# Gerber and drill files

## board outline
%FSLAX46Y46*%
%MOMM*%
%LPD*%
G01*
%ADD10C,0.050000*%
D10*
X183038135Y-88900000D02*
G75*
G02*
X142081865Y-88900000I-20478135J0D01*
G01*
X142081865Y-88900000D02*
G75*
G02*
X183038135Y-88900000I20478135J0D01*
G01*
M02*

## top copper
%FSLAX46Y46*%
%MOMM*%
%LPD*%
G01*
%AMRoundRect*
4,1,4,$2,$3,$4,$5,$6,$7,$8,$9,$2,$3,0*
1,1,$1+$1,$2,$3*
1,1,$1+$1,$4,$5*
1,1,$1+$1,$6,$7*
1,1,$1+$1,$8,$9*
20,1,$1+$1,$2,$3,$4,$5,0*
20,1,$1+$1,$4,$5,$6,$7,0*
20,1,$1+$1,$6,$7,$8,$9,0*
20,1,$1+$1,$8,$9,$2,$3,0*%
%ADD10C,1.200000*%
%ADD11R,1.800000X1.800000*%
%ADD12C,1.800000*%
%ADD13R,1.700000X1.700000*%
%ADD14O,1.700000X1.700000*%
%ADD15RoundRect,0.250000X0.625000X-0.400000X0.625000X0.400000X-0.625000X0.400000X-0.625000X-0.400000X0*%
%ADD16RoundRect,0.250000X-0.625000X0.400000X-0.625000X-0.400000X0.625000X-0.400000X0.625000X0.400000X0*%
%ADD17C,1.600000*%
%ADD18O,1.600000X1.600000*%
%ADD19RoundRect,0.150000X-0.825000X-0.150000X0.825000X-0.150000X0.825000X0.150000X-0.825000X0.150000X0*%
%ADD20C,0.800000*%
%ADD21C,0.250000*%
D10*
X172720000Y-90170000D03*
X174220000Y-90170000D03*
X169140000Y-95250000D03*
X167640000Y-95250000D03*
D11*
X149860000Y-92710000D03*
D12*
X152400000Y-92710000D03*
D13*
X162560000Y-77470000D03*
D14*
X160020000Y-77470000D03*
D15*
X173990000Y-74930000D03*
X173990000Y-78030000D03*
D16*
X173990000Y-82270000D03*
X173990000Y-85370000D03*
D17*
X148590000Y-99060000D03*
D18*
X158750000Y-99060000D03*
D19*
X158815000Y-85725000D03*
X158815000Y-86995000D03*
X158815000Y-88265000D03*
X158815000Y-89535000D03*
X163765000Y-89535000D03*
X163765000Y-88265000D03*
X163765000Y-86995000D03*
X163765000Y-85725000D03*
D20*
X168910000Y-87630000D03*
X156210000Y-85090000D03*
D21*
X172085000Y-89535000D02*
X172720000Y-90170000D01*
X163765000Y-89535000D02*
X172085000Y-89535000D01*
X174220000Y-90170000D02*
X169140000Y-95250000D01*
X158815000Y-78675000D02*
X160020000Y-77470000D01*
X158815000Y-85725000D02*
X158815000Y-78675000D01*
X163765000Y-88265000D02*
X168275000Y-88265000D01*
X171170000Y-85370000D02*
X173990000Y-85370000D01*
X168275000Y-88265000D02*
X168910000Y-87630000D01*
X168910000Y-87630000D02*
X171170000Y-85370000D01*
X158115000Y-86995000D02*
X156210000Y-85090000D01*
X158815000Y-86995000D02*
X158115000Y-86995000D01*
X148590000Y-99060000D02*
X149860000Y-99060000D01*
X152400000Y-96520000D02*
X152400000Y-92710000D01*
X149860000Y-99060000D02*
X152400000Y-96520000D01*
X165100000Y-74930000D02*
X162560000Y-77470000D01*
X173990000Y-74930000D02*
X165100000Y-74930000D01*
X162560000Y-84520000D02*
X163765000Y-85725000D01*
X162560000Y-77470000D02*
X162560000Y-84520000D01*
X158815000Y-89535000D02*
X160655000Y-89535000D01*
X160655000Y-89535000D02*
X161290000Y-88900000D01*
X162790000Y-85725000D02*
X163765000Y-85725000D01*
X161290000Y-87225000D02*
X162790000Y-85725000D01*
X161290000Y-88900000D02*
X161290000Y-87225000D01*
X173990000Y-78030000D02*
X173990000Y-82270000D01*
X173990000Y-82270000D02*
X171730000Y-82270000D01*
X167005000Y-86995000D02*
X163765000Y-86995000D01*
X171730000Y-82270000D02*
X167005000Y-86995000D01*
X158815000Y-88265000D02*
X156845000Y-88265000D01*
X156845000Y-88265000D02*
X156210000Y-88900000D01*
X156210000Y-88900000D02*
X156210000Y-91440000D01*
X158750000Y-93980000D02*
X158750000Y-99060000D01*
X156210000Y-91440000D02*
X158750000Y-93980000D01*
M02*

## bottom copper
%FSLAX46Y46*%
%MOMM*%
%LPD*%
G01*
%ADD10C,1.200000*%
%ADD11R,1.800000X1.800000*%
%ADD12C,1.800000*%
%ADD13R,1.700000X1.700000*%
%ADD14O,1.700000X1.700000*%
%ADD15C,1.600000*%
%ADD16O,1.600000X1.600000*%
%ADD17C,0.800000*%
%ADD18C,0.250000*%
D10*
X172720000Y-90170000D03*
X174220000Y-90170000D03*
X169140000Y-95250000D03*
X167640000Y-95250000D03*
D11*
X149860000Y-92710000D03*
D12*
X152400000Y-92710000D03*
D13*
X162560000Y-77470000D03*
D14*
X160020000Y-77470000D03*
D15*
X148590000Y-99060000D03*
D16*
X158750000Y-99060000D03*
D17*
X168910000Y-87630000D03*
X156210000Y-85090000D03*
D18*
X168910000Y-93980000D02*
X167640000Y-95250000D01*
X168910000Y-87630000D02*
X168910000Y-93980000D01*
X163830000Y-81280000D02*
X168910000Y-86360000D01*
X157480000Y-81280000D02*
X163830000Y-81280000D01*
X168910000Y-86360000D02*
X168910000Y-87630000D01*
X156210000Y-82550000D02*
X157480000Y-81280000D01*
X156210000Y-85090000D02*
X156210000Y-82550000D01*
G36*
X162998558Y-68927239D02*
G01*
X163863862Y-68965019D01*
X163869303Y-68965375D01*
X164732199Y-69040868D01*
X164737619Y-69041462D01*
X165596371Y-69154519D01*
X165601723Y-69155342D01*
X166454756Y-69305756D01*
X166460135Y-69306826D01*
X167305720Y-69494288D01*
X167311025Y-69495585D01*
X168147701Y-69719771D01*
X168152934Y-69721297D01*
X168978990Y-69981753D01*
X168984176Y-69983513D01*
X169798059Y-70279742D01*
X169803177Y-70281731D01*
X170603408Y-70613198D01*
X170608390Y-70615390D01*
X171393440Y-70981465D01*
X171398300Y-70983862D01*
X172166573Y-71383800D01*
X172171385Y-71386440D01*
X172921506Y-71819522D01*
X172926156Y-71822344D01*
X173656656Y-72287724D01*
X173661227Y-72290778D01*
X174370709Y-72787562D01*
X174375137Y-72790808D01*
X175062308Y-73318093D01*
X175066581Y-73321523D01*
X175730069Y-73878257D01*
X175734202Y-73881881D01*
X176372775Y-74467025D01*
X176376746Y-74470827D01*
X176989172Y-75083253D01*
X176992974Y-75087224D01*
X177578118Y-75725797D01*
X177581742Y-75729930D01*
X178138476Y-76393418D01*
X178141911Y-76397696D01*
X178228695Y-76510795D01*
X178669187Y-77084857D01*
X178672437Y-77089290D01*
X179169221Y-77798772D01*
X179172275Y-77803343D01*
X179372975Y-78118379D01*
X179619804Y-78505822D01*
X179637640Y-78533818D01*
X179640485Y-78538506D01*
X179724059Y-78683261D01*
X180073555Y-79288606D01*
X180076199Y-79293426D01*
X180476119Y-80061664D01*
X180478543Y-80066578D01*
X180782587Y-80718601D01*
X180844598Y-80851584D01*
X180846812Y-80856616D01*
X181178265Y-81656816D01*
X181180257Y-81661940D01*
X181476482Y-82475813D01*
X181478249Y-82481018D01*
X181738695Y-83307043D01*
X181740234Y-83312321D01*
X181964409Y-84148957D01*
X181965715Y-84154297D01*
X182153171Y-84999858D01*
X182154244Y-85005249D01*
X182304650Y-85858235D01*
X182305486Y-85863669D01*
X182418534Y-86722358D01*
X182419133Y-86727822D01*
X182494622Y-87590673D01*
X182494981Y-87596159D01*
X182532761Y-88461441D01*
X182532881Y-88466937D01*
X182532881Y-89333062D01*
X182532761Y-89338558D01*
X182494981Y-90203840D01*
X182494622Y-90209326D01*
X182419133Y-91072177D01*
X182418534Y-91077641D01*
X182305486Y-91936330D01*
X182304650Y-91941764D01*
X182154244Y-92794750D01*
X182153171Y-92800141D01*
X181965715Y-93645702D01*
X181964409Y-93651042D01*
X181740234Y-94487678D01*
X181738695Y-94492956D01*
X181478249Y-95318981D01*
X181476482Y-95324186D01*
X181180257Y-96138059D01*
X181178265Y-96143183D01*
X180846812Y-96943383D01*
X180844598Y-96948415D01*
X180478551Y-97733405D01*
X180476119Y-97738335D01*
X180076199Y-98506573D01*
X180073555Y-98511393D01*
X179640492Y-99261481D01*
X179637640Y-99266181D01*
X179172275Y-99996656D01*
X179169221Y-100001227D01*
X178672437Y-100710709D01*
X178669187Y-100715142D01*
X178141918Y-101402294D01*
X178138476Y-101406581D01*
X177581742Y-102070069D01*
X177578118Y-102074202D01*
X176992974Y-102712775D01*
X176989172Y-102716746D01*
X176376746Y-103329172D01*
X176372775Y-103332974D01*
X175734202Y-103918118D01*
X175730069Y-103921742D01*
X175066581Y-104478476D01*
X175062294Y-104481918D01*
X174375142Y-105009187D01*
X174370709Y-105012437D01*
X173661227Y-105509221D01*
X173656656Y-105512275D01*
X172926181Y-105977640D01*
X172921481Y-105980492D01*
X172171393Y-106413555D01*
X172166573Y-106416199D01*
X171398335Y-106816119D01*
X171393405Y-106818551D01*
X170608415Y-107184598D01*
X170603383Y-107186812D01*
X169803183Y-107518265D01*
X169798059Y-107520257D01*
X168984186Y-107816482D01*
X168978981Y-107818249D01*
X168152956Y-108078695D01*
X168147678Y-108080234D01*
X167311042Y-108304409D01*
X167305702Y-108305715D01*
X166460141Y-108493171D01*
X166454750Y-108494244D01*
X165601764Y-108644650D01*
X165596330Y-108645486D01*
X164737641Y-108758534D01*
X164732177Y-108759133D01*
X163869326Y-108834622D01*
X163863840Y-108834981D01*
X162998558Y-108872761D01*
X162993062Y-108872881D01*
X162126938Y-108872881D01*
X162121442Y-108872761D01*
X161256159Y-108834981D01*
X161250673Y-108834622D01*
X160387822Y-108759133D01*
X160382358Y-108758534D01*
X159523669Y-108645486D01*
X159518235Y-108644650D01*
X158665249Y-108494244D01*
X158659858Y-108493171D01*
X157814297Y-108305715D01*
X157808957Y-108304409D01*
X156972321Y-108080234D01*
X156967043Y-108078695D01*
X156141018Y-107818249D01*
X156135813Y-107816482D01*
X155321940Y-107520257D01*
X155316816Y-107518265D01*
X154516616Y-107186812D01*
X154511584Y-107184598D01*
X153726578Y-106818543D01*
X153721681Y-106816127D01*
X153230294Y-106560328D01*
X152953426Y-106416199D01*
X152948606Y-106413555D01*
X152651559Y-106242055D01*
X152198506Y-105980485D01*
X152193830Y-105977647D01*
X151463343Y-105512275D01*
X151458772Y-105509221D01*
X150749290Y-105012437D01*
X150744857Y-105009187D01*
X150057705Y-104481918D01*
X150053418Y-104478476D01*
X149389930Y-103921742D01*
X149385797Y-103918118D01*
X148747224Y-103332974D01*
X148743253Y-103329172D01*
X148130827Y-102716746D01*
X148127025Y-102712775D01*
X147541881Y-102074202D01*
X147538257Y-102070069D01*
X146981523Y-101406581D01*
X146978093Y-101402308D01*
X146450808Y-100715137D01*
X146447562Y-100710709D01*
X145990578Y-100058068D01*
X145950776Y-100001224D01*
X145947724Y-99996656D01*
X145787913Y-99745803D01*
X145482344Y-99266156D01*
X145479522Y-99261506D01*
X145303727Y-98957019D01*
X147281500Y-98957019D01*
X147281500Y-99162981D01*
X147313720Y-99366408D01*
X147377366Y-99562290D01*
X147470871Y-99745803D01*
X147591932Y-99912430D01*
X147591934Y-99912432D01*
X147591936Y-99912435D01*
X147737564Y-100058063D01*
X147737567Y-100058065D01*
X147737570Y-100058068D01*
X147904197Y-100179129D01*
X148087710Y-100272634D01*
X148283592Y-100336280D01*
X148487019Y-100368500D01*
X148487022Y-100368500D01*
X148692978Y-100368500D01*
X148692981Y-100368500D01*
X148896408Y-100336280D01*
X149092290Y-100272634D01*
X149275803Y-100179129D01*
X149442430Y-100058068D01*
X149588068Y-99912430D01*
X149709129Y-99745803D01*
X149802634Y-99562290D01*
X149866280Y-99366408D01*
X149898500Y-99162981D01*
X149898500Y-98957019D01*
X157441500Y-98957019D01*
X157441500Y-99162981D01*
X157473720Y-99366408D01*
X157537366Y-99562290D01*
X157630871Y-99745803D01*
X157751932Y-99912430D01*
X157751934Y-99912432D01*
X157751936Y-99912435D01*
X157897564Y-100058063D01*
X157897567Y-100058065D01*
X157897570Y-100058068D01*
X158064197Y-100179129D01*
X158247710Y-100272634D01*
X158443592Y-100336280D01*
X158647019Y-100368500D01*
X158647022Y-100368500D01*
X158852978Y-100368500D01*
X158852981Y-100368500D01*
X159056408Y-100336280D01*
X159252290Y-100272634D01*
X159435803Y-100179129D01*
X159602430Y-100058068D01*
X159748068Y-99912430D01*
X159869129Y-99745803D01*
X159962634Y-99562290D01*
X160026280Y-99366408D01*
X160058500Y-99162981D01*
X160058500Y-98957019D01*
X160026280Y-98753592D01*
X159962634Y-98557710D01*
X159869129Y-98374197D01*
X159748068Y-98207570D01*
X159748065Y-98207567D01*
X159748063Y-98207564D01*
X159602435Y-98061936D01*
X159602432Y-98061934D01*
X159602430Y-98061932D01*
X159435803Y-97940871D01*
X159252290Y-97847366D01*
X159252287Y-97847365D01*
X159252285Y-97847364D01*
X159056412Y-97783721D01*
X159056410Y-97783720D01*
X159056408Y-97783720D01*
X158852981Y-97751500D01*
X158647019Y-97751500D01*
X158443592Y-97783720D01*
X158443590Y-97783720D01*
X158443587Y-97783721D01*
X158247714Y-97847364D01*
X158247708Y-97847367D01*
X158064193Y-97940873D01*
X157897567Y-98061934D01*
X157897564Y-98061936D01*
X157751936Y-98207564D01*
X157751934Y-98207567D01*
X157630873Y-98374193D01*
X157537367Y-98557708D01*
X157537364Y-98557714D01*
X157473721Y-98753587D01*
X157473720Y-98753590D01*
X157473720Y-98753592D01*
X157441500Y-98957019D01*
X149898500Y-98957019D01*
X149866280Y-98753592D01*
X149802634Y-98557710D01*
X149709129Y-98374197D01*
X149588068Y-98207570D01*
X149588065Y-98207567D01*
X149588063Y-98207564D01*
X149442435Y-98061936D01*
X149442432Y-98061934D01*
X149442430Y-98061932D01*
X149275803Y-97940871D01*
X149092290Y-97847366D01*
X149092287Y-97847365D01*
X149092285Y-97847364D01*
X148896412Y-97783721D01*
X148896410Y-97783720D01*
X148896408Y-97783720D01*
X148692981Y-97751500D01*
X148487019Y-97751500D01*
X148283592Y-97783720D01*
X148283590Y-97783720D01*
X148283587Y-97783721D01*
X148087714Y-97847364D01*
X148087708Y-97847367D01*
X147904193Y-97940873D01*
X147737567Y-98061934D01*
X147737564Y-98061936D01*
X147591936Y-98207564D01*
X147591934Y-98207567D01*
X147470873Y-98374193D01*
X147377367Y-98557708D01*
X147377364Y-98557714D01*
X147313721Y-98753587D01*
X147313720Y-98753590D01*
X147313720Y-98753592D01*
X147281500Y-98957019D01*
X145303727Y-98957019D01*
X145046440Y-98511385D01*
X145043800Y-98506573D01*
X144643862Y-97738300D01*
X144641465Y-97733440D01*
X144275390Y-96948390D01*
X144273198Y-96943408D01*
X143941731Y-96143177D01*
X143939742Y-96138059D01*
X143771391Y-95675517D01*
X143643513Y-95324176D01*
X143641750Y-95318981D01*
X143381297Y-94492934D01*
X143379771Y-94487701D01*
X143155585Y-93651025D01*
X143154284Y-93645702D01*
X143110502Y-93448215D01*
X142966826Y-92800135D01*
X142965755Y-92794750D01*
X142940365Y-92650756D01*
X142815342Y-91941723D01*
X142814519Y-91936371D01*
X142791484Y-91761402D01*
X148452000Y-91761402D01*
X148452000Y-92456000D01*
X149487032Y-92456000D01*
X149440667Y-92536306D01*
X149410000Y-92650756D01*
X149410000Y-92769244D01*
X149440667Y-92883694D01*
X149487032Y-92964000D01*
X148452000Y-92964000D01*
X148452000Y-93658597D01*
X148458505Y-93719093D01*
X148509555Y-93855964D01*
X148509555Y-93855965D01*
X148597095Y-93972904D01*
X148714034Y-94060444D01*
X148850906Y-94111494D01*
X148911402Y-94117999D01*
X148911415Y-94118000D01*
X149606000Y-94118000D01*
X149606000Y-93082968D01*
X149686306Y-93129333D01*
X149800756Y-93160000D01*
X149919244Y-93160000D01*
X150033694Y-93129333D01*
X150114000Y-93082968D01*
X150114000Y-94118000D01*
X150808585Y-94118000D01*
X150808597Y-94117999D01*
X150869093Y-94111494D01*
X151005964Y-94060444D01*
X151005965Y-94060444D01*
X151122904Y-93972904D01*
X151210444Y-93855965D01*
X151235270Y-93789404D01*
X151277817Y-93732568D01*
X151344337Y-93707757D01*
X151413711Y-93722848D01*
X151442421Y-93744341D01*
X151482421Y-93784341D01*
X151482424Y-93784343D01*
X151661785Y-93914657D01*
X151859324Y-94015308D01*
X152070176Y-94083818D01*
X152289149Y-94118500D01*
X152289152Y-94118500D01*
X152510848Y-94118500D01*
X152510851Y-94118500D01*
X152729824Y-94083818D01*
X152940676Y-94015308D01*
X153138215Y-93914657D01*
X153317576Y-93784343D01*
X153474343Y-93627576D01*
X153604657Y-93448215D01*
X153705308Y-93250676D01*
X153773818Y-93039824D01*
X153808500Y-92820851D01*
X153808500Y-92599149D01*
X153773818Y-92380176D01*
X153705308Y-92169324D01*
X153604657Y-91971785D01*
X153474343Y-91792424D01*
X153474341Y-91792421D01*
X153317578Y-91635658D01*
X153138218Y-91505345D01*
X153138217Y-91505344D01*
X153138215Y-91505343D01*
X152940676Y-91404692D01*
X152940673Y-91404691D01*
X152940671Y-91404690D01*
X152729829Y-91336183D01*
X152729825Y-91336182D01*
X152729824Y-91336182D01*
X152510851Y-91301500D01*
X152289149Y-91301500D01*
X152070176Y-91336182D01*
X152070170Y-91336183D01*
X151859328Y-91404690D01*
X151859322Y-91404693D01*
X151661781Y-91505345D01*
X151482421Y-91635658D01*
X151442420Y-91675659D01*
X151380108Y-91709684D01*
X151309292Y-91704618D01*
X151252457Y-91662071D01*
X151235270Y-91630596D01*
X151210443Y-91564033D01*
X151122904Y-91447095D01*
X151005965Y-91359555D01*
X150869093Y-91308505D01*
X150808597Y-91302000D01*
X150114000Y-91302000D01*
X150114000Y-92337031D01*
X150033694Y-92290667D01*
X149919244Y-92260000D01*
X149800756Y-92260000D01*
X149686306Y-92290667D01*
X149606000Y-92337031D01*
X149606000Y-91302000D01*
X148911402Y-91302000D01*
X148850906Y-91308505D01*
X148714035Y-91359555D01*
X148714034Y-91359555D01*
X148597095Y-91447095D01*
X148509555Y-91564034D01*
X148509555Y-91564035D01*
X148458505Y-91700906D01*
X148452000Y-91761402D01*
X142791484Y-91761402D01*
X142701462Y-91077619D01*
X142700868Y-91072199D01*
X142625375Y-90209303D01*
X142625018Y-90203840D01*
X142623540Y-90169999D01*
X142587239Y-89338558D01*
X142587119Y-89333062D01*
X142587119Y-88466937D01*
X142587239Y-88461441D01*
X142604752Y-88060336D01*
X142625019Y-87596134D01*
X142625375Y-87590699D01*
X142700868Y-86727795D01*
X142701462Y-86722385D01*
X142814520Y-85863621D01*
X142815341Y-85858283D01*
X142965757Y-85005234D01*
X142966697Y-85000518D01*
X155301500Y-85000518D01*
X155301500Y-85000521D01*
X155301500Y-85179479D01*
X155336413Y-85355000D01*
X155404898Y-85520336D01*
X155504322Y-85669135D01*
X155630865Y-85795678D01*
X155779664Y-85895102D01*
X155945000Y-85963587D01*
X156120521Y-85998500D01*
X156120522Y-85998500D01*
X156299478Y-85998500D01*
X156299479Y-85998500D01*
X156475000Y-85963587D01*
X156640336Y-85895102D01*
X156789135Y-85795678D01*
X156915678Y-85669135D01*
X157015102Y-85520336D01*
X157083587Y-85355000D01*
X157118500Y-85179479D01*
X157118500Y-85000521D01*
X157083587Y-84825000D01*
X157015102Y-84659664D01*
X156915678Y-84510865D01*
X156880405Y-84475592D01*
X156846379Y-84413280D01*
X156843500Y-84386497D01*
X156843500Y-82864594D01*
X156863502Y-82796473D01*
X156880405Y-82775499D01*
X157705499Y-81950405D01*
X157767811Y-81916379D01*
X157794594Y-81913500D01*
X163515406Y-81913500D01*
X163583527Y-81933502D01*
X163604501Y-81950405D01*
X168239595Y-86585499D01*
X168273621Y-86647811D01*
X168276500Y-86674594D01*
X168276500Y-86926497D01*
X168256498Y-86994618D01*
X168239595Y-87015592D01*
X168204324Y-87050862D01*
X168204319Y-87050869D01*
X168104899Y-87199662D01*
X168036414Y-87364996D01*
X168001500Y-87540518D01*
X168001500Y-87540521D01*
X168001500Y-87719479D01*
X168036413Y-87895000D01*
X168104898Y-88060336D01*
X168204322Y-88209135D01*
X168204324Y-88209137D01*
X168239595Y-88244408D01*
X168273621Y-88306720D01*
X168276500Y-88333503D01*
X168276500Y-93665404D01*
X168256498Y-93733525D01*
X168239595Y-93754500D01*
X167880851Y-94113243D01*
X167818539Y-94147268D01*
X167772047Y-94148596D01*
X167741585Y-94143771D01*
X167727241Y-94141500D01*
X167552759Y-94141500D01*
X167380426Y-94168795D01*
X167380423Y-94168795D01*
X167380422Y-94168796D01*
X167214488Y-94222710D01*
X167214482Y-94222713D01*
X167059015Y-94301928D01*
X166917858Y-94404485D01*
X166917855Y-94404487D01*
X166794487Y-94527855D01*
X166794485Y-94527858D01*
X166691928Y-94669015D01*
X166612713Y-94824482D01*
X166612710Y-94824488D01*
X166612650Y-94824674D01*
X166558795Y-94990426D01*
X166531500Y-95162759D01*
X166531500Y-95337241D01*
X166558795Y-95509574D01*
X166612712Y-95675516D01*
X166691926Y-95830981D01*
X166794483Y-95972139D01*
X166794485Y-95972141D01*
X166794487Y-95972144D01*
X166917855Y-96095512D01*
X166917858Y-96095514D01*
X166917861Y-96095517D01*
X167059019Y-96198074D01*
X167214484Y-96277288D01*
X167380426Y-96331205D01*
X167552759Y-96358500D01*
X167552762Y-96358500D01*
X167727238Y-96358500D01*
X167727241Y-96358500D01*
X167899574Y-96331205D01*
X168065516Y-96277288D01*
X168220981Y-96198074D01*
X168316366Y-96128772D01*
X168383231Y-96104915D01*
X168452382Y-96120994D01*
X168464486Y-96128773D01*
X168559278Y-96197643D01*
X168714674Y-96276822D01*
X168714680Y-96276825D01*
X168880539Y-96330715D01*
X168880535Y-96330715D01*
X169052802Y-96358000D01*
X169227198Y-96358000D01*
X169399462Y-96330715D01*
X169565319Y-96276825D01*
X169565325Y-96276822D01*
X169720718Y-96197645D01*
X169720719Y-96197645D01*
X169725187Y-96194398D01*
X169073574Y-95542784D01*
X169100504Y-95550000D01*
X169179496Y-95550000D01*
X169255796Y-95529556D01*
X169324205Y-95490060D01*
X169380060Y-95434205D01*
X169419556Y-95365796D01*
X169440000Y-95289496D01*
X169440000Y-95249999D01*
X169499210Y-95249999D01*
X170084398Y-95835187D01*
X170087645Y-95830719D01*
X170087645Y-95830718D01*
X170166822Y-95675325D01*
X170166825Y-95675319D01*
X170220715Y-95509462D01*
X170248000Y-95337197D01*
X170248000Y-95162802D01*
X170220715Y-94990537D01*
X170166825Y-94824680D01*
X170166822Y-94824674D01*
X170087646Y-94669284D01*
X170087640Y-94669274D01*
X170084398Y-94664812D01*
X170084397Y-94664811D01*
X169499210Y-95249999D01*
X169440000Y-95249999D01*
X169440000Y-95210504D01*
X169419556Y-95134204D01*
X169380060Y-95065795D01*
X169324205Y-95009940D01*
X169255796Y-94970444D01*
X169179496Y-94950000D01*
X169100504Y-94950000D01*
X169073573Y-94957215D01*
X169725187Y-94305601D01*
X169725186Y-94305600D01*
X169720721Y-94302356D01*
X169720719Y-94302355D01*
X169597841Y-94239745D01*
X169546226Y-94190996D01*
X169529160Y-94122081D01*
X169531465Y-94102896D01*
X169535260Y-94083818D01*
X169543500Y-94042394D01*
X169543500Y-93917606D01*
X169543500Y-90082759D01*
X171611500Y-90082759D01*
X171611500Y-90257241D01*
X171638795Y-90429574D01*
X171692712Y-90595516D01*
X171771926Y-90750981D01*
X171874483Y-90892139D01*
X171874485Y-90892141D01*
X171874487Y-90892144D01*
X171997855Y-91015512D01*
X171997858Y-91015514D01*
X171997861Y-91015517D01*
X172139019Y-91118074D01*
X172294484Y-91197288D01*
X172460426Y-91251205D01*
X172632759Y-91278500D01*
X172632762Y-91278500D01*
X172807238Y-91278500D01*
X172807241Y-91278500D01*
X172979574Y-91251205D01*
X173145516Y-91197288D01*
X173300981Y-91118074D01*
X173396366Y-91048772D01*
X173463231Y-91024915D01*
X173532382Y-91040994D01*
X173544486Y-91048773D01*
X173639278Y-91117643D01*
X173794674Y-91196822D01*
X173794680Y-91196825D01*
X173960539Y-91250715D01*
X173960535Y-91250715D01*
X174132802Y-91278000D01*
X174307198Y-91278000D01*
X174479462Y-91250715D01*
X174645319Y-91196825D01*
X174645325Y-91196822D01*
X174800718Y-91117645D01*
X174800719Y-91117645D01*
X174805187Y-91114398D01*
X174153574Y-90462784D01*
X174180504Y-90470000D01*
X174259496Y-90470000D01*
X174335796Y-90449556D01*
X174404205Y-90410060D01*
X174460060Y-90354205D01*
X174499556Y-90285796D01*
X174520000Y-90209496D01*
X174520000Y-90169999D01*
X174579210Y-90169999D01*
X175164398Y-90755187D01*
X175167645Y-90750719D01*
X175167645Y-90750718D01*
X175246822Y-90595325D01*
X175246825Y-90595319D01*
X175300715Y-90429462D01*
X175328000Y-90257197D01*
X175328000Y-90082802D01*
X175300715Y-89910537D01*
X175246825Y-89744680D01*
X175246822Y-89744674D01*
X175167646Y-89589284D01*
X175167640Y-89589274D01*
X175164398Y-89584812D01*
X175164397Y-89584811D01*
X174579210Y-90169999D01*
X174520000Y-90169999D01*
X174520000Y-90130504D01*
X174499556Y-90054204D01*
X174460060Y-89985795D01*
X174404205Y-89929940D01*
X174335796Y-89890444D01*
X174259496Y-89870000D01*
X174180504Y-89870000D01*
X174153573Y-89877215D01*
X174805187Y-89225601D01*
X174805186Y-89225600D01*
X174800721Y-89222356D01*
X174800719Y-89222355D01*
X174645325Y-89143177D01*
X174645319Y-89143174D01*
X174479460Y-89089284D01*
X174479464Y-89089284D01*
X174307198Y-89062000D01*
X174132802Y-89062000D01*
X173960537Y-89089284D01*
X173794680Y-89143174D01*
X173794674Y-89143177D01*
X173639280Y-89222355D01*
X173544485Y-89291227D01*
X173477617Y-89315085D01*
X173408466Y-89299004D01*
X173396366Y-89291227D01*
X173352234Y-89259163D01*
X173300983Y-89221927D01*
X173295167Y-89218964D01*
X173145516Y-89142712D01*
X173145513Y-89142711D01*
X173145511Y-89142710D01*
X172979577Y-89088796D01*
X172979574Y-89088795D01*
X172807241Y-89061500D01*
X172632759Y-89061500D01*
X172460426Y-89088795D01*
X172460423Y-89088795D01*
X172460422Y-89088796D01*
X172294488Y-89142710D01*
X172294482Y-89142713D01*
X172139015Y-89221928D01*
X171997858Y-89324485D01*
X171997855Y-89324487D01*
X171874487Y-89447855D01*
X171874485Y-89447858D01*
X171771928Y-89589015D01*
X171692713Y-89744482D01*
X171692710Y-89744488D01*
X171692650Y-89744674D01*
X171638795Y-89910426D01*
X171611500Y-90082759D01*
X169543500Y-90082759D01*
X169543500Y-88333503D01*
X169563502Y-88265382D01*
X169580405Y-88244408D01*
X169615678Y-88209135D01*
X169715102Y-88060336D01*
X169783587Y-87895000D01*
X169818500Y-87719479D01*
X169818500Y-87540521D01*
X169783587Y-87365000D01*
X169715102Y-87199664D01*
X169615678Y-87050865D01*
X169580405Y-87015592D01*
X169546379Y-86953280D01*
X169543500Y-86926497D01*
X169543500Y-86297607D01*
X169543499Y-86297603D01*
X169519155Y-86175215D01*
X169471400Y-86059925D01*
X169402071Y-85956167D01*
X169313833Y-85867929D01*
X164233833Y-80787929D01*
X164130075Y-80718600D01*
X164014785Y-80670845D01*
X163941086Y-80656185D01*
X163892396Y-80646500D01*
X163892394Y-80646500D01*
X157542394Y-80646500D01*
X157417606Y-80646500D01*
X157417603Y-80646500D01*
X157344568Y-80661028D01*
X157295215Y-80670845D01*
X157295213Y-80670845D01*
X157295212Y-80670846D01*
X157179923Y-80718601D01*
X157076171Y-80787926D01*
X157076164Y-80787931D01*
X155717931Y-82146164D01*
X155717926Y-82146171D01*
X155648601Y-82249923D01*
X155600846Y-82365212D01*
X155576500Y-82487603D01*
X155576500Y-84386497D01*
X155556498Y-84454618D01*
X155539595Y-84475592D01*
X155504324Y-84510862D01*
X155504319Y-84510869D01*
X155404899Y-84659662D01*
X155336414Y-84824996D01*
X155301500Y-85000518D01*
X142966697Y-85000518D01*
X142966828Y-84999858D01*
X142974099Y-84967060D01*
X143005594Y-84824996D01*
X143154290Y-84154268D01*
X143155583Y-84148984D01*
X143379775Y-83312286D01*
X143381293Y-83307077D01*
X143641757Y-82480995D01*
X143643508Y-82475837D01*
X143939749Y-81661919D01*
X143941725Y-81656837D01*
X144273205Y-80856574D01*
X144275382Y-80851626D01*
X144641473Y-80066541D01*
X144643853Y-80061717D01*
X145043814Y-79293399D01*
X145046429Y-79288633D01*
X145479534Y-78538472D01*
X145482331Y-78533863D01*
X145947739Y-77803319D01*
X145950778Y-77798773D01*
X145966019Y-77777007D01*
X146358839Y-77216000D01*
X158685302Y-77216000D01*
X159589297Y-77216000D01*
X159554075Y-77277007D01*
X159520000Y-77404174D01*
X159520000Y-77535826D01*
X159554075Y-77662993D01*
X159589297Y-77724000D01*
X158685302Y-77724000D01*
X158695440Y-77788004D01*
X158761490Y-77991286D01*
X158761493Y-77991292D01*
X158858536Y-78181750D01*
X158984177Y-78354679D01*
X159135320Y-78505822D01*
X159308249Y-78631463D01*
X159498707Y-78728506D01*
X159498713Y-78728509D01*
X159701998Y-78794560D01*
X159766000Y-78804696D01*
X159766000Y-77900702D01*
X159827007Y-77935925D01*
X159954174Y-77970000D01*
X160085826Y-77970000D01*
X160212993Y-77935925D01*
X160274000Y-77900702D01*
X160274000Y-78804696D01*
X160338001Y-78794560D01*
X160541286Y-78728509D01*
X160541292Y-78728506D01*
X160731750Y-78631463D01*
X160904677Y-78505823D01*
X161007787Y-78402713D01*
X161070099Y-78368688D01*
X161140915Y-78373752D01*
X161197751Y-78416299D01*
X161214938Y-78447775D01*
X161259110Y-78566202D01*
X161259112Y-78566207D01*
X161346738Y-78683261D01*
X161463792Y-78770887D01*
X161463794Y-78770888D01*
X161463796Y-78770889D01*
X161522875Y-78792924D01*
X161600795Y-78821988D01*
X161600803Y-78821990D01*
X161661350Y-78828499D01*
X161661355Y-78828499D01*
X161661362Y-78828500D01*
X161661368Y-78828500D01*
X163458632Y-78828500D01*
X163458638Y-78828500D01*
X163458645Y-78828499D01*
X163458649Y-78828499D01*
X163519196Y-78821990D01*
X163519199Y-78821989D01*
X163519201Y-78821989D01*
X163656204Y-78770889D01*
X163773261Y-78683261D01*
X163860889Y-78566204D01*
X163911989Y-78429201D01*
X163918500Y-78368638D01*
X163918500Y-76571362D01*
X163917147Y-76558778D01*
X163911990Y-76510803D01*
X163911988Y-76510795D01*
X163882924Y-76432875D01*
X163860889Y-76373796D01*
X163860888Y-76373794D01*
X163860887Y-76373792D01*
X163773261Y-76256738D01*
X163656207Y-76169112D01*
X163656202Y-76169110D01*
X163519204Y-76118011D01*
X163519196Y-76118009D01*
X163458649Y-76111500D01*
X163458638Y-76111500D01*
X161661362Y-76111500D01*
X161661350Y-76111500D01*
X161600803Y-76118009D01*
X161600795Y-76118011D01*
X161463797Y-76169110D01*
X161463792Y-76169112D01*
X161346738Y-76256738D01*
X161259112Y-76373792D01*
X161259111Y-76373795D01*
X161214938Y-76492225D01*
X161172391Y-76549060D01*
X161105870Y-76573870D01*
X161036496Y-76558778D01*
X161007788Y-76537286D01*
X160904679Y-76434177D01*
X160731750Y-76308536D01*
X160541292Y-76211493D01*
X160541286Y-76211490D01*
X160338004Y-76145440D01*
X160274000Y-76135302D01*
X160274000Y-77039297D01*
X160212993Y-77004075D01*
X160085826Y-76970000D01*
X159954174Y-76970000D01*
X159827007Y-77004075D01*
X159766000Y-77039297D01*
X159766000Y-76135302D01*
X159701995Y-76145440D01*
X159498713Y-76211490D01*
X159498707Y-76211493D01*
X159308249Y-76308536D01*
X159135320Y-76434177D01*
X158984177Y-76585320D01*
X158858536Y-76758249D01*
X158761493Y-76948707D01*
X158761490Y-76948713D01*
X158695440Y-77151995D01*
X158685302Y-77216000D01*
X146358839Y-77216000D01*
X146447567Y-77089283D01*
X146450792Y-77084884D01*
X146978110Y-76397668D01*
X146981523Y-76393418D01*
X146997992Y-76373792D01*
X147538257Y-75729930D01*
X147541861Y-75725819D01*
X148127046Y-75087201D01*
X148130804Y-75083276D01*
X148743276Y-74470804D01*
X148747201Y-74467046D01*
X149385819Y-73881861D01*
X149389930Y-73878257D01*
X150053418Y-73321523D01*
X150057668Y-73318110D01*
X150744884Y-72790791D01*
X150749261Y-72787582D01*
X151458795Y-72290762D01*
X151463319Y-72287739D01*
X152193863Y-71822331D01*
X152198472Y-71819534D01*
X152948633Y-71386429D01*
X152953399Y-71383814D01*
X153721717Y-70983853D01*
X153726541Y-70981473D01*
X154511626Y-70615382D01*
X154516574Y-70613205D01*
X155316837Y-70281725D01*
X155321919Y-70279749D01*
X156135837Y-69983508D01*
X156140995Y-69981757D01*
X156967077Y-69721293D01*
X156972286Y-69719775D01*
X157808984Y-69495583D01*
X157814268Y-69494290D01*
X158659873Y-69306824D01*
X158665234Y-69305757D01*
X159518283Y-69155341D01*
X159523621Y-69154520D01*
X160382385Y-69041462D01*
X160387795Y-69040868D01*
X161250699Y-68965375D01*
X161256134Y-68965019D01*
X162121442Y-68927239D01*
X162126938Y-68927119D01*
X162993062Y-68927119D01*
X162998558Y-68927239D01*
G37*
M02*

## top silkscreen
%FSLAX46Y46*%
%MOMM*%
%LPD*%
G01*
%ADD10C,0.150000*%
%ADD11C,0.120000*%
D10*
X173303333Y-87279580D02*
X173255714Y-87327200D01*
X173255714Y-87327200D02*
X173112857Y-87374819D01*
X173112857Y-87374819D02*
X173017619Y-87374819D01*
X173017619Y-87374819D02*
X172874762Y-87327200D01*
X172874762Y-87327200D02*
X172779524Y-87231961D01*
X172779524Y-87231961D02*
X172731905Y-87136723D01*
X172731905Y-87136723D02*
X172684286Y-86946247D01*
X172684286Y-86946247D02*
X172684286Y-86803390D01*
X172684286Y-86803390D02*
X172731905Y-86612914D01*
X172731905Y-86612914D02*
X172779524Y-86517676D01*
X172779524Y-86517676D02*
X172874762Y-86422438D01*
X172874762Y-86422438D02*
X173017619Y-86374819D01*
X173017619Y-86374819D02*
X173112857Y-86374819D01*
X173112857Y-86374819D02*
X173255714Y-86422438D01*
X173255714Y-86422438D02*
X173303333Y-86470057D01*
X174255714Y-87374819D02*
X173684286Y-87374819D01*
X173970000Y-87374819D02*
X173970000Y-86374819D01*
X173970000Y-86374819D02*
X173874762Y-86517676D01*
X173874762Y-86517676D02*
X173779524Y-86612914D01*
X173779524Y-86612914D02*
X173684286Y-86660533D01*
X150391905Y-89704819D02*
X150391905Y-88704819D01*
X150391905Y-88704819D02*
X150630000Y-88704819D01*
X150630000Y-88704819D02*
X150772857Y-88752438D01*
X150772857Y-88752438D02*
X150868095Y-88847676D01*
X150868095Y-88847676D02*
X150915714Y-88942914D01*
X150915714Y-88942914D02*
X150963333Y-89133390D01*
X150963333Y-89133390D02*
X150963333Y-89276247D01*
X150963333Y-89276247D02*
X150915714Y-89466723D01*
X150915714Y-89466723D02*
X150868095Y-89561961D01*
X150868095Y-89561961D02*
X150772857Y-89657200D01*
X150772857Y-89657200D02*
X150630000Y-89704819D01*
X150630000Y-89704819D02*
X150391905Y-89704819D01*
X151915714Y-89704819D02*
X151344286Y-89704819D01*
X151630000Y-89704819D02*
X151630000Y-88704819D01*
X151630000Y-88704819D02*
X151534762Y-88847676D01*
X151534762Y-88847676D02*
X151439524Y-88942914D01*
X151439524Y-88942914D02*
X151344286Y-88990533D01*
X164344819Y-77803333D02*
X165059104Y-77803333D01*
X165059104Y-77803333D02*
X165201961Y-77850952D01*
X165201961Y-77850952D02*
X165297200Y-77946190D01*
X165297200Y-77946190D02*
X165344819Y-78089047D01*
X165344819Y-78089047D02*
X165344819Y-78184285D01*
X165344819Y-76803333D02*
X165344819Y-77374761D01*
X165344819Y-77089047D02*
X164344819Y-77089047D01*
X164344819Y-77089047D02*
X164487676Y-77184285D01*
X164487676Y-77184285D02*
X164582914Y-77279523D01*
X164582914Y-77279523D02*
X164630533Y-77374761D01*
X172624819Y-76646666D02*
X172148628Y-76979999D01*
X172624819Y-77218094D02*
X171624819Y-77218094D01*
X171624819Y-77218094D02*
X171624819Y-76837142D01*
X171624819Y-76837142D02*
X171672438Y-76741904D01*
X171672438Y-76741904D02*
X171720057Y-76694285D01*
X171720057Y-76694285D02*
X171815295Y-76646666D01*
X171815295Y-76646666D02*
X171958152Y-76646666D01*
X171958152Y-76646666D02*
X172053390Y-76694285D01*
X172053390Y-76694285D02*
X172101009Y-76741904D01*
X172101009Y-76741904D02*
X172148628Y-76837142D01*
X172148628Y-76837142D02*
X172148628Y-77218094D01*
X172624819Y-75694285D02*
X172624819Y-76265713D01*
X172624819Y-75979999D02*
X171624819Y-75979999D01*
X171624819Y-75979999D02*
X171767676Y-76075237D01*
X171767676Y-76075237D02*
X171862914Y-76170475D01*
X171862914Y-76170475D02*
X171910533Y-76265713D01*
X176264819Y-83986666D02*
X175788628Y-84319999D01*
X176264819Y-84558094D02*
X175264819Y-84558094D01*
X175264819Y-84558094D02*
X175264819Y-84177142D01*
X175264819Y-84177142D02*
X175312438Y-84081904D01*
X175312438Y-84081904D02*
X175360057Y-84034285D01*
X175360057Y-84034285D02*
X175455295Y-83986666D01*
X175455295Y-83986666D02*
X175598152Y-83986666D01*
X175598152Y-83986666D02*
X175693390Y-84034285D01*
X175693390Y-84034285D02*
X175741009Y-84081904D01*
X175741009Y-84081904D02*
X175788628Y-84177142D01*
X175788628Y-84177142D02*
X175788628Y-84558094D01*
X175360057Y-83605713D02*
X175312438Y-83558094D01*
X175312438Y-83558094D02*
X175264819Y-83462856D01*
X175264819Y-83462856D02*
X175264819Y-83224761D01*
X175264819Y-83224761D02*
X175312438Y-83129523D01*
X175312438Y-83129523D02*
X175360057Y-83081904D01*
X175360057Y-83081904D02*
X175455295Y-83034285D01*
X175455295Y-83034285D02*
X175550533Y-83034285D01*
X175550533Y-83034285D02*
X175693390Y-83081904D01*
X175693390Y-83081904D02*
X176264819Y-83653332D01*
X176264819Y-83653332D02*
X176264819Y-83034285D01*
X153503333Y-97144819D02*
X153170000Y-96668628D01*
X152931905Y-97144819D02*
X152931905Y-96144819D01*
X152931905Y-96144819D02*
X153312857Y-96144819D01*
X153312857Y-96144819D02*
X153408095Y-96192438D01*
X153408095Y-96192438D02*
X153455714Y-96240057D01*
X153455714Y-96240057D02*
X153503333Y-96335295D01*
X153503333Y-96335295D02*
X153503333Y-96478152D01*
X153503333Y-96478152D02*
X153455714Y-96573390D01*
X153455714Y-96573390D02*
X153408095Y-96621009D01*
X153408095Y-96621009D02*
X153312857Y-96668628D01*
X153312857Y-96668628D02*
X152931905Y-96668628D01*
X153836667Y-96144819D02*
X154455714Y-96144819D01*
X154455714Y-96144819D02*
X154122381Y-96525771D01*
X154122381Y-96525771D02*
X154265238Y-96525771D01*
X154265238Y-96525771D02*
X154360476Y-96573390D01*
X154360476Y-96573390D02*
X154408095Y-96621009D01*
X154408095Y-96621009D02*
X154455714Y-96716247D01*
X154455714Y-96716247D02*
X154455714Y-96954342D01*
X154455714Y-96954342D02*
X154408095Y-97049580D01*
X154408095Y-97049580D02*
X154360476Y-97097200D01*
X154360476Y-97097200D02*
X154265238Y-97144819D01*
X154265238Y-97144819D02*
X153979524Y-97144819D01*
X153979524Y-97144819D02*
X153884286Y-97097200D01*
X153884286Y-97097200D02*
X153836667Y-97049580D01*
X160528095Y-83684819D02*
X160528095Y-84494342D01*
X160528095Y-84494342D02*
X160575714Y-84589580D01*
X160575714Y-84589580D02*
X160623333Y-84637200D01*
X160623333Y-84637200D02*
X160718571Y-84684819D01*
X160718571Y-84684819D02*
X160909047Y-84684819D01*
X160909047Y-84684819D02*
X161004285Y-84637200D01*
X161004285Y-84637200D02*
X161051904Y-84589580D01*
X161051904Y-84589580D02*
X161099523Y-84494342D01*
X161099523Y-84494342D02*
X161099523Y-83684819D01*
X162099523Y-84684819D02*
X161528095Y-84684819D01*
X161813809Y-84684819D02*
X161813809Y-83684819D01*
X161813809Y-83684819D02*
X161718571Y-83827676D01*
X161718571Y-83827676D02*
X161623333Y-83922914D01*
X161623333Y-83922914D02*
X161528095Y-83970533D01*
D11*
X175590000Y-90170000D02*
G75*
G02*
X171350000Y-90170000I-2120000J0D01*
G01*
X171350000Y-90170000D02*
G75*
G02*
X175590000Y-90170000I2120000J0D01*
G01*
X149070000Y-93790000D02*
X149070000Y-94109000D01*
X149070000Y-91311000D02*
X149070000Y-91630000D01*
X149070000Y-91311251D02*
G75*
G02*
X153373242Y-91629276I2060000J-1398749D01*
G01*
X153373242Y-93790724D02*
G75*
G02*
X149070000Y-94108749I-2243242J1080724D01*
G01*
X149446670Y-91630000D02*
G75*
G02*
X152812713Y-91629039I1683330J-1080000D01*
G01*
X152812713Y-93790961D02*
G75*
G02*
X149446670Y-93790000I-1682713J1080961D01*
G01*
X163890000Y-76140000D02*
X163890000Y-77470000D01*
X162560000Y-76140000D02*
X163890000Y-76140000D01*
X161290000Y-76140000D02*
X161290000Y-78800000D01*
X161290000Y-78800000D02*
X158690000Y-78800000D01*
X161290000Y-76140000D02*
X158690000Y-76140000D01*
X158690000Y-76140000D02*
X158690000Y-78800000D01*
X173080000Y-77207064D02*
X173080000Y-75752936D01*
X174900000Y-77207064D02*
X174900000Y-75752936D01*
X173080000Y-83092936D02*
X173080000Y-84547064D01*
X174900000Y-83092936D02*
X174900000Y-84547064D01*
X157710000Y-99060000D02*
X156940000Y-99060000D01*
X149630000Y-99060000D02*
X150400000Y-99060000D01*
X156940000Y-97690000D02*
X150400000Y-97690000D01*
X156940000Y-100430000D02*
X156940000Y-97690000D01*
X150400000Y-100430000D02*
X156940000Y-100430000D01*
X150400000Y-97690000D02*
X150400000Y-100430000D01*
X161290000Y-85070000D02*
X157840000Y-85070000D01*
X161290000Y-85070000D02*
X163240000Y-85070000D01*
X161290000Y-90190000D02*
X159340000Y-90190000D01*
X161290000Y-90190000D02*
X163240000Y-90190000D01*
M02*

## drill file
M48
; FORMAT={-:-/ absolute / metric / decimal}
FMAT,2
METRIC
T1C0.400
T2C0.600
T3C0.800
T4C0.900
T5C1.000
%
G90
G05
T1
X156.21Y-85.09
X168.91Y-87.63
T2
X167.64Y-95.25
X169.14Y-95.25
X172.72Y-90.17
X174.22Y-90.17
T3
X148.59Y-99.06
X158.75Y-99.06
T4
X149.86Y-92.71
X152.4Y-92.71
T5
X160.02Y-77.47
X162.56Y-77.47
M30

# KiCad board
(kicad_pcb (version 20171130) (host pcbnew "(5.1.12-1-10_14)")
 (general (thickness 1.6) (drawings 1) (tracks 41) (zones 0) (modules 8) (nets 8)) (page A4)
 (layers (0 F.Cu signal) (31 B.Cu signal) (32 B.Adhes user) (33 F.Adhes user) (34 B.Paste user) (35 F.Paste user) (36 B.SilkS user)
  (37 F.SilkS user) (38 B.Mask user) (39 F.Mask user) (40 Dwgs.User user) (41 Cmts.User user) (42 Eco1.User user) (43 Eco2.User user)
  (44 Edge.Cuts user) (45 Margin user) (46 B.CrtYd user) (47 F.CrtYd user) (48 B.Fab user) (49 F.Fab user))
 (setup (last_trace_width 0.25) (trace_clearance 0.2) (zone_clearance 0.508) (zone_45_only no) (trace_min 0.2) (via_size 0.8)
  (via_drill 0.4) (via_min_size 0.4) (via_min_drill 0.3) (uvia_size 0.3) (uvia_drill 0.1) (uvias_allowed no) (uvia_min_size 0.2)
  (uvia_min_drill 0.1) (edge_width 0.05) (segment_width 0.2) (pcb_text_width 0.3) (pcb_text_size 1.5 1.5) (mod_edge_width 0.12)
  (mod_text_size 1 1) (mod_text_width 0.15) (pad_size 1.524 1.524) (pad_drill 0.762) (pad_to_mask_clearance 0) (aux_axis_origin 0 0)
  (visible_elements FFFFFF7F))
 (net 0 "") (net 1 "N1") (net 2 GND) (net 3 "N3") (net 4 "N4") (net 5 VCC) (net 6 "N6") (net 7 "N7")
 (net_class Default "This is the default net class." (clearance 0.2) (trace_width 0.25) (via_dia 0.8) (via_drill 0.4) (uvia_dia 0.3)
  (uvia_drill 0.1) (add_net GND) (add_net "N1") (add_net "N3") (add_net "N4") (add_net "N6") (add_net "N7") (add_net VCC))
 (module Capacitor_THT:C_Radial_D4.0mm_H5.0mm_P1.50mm (layer F.Cu) (at 172.72 90.17)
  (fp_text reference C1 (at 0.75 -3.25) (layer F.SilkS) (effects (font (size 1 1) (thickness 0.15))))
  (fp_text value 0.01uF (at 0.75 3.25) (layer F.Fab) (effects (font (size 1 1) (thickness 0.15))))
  (fp_circle (center 0.75 0) (end 2.87 0) (layer F.SilkS) (width 0.12))
  (pad 1 thru_hole circle (at 0 0) (size 1.2 1.2) (drill 0.6) (layers *.Cu *.Mask) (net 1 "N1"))
  (pad 2 thru_hole circle (at 1.5 0) (size 1.2 1.2) (drill 0.6) (layers *.Cu *.Mask) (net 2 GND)))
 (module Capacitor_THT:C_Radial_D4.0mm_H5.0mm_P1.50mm (layer B.Cu) (at 167.64 95.25)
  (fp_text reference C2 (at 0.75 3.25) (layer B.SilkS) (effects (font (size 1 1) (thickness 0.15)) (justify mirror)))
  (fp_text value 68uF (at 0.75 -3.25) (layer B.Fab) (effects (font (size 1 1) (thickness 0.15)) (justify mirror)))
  (pad 2 thru_hole circle (at 1.5 0) (size 1.2 1.2) (drill 0.6) (layers *.Cu *.Mask) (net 2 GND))
  (pad 1 thru_hole circle (at 0 0) (size 1.2 1.2) (drill 0.6) (layers *.Cu *.Mask) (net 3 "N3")))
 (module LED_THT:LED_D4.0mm (layer F.Cu) (at 149.86 92.71)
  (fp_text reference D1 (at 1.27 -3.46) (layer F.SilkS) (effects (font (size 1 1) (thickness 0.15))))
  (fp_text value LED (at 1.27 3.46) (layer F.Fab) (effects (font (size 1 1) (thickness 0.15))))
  (fp_line (start -0.79 1.08) (end -0.79 1.399) (layer F.SilkS) (width 0.12))
  (fp_line (start -0.79 -1.399) (end -0.79 -1.08) (layer F.SilkS) (width 0.12))
  (fp_arc (start 1.27 0) (end -0.79 -1.398749) (angle 120.1) (layer F.SilkS) (width 0.12))
  (fp_arc (start 1.27 0) (end -0.79 1.398749) (angle -120.1) (layer F.SilkS) (width 0.12))
  (fp_arc (start 1.27 0) (end -0.41333 -1.08) (angle 114.6) (layer F.SilkS) (width 0.12))
  (fp_arc (start 1.27 0) (end -0.41333 1.08) (angle -114.6) (layer F.SilkS) (width 0.12))
  (pad 1 thru_hole rect (at 0 0) (size 1.8 1.8) (drill 0.9) (layers *.Cu *.Mask) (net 2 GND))
  (pad 2 thru_hole circle (at 2.54 0) (size 1.8 1.8) (drill 0.9) (layers *.Cu *.Mask) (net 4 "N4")))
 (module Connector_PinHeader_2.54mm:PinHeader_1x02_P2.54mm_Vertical (layer F.Cu) (at 162.56 77.47 270)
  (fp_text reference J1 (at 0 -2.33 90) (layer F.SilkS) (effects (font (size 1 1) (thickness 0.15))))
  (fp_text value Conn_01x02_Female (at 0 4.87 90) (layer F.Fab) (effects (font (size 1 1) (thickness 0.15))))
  (fp_line (start -1.33 -1.33) (end 0 -1.33) (layer F.SilkS) (width 0.12))
  (fp_line (start -1.33 0) (end -1.33 -1.33) (layer F.SilkS) (width 0.12))
  (fp_line (start -1.33 1.27) (end 1.33 1.27) (layer F.SilkS) (width 0.12))
  (fp_line (start 1.33 1.27) (end 1.33 3.87) (layer F.SilkS) (width 0.12))
  (fp_line (start -1.33 1.27) (end -1.33 3.87) (layer F.SilkS) (width 0.12))
  (fp_line (start -1.33 3.87) (end 1.33 3.87) (layer F.SilkS) (width 0.12))
  (pad 1 thru_hole rect (at 0 0 270) (size 1.7 1.7) (drill 1) (layers *.Cu *.Mask) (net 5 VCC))
  (pad 2 thru_hole oval (at 0 2.54 270) (size 1.7 1.7) (drill 1) (layers *.Cu *.Mask) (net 2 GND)))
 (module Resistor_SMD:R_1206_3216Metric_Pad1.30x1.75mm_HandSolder (layer F.Cu) (at 173.99 76.48 90)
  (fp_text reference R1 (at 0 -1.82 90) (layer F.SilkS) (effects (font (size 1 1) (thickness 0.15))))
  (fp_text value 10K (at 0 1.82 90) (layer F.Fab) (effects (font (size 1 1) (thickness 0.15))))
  (fp_line (start -0.727064 -0.91) (end 0.727064 -0.91) (layer F.SilkS) (width 0.12))
  (fp_line (start -0.727064 0.91) (end 0.727064 0.91) (layer F.SilkS) (width 0.12))
  (pad 2 smd roundrect (at 1.55 0 90) (size 1.3 1.75) (layers F.Cu F.Paste F.Mask) (roundrect_rratio 0.192308) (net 5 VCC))
  (pad 1 smd roundrect (at -1.55 0 90) (size 1.3 1.75) (layers F.Cu F.Paste F.Mask) (roundrect_rratio 0.192308) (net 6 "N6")))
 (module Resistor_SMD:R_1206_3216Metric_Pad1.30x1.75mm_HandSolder (layer F.Cu) (at 173.99 83.82 270)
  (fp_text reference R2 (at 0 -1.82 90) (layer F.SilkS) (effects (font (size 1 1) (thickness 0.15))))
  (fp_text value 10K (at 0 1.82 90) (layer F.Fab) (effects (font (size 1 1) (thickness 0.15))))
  (fp_line (start -0.727064 0.91) (end 0.727064 0.91) (layer F.SilkS) (width 0.12))
  (fp_line (start -0.727064 -0.91) (end 0.727064 -0.91) (layer F.SilkS) (width 0.12))
  (pad 1 smd roundrect (at -1.55 0 270) (size 1.3 1.75) (layers F.Cu F.Paste F.Mask) (roundrect_rratio 0.192308) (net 6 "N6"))
  (pad 2 smd roundrect (at 1.55 0 270) (size 1.3 1.75) (layers F.Cu F.Paste F.Mask) (roundrect_rratio 0.192308) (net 3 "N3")))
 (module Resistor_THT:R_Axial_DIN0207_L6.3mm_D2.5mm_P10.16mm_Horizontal (layer F.Cu) (at 148.59 99.06)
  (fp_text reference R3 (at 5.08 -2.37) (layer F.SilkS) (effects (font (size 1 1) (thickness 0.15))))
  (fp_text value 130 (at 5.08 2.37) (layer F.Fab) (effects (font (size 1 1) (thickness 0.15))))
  (fp_line (start 9.12 0) (end 8.35 0) (layer F.SilkS) (width 0.12))
  (fp_line (start 1.04 0) (end 1.81 0) (layer F.SilkS) (width 0.12))
  (fp_line (start 8.35 -1.37) (end 1.81 -1.37) (layer F.SilkS) (width 0.12))
  (fp_line (start 8.35 1.37) (end 8.35 -1.37) (layer F.SilkS) (width 0.12))
  (fp_line (start 1.81 1.37) (end 8.35 1.37) (layer F.SilkS) (width 0.12))
  (fp_line (start 1.81 -1.37) (end 1.81 1.37) (layer F.SilkS) (width 0.12))
  (pad 1 thru_hole circle (at 0 0) (size 1.6 1.6) (drill 0.8) (layers *.Cu *.Mask) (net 4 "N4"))
  (pad 2 thru_hole oval (at 10.16 0) (size 1.6 1.6) (drill 0.8) (layers *.Cu *.Mask) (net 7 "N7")))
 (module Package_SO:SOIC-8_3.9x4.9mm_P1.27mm (layer F.Cu) (at 161.29 87.63)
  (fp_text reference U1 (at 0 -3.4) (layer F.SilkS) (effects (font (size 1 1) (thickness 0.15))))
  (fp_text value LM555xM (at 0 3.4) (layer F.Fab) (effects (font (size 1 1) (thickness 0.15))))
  (fp_line (start 0 -2.56) (end -3.45 -2.56) (layer F.SilkS) (width 0.12))
  (fp_line (start 0 -2.56) (end 1.95 -2.56) (layer F.SilkS) (width 0.12))
  (fp_line (start 0 2.56) (end -1.95 2.56) (layer F.SilkS) (width 0.12))
  (fp_line (start 0 2.56) (end 1.95 2.56) (layer F.SilkS) (width 0.12))
  (pad 1 smd roundrect (at -2.475 -1.905) (size 1.95 0.6) (layers F.Cu F.Paste F.Mask) (roundrect_rratio 0.25) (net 2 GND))
  (pad 2 smd roundrect (at -2.475 -0.635) (size 1.95 0.6) (layers F.Cu F.Paste F.Mask) (roundrect_rratio 0.25) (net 3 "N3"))
  (pad 3 smd roundrect (at -2.475 0.635) (size 1.95 0.6) (layers F.Cu F.Paste F.Mask) (roundrect_rratio 0.25) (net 7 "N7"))
  (pad 4 smd roundrect (at -2.475 1.905) (size 1.95 0.6) (layers F.Cu F.Paste F.Mask) (roundrect_rratio 0.25) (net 5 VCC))
  (pad 5 smd roundrect (at 2.475 1.905) (size 1.95 0.6) (layers F.Cu F.Paste F.Mask) (roundrect_rratio 0.25) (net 1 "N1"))
  (pad 6 smd roundrect (at 2.475 0.635) (size 1.95 0.6) (layers F.Cu F.Paste F.Mask) (roundrect_rratio 0.25) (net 3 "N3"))
  (pad 7 smd roundrect (at 2.475 -0.635) (size 1.95 0.6) (layers F.Cu F.Paste F.Mask) (roundrect_rratio 0.25) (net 6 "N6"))
  (pad 8 smd roundrect (at 2.475 -1.905) (size 1.95 0.6) (layers F.Cu F.Paste F.Mask) (roundrect_rratio 0.25) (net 5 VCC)))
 (gr_circle (center 162.56 88.9) (end 182.88 91.44) (layer Edge.Cuts) (width 0.05))
 (segment (start 172.085 89.535) (end 172.72 90.17) (width 0.25) (layer F.Cu) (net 1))
 (segment (start 163.765 89.535) (end 172.085 89.535) (width 0.25) (layer F.Cu) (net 1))
 (segment (start 174.22 90.17) (end 169.14 95.25) (width 0.25) (layer F.Cu) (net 2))
 (segment (start 158.815 78.675) (end 160.02 77.47) (width 0.25) (layer F.Cu) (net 2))
 (segment (start 158.815 85.725) (end 158.815 78.675) (width 0.25) (layer F.Cu) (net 2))
 (segment (start 163.765 88.265) (end 168.275 88.265) (width 0.25) (layer F.Cu) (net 3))
 (segment (start 171.17 85.37) (end 173.99 85.37) (width 0.25) (layer F.Cu) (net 3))
 (segment (start 168.275 88.265) (end 168.91 87.63) (width 0.25) (layer F.Cu) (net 3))
 (segment (start 168.91 87.63) (end 171.17 85.37) (width 0.25) (layer F.Cu) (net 3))
 (via (at 168.91 87.63) (size 0.8) (drill 0.4) (layers F.Cu B.Cu) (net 3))
 (segment (start 168.91 93.98) (end 167.64 95.25) (width 0.25) (layer B.Cu) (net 3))
 (segment (start 168.91 87.63) (end 168.91 93.98) (width 0.25) (layer B.Cu) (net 3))
 (via (at 156.21 85.09) (size 0.8) (drill 0.4) (layers F.Cu B.Cu) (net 3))
 (segment (start 158.115 86.995) (end 156.21 85.09) (width 0.25) (layer F.Cu) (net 3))
 (segment (start 158.815 86.995) (end 158.115 86.995) (width 0.25) (layer F.Cu) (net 3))
 (segment (start 163.83 81.28) (end 168.91 86.36) (width 0.25) (layer B.Cu) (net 3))
 (segment (start 157.48 81.28) (end 163.83 81.28) (width 0.25) (layer B.Cu) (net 3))
 (segment (start 168.91 86.36) (end 168.91 87.63) (width 0.25) (layer B.Cu) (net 3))
 (segment (start 156.21 82.55) (end 157.48 81.28) (width 0.25) (layer B.Cu) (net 3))
 (segment (start 156.21 85.09) (end 156.21 82.55) (width 0.25) (layer B.Cu) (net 3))
 (segment (start 148.59 99.06) (end 149.86 99.06) (width 0.25) (layer F.Cu) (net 4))
 (segment (start 152.4 96.52) (end 152.4 92.71) (width 0.25) (layer F.Cu) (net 4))
 (segment (start 149.86 99.06) (end 152.4 96.52) (width 0.25) (layer F.Cu) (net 4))
 (segment (start 165.1 74.93) (end 162.56 77.47) (width 0.25) (layer F.Cu) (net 5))
 (segment (start 173.99 74.93) (end 165.1 74.93) (width 0.25) (layer F.Cu) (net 5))
 (segment (start 162.56 84.52) (end 163.765 85.725) (width 0.25) (layer F.Cu) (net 5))
 (segment (start 162.56 77.47) (end 162.56 84.52) (width 0.25) (layer F.Cu) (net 5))
 (segment (start 158.815 89.535) (end 160.655 89.535) (width 0.25) (layer F.Cu) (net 5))
 (segment (start 160.655 89.535) (end 161.29 88.9) (width 0.25) (layer F.Cu) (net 5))
 (segment (start 162.79 85.725) (end 163.765 85.725) (width 0.25) (layer F.Cu) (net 5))
 (segment (start 161.29 87.225) (end 162.79 85.725) (width 0.25) (layer F.Cu) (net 5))
 (segment (start 161.29 88.9) (end 161.29 87.225) (width 0.25) (layer F.Cu) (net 5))
 (segment (start 173.99 78.03) (end 173.99 82.27) (width 0.25) (layer F.Cu) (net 6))
 (segment (start 173.99 82.27) (end 171.73 82.27) (width 0.25) (layer F.Cu) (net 6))
 (segment (start 167.005 86.995) (end 163.765 86.995) (width 0.25) (layer F.Cu) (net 6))
 (segment (start 171.73 82.27) (end 167.005 86.995) (width 0.25) (layer F.Cu) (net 6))
 (segment (start 158.815 88.265) (end 156.845 88.265) (width 0.25) (layer F.Cu) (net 7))
 (segment (start 156.845 88.265) (end 156.21 88.9) (width 0.25) (layer F.Cu) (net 7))
 (segment (start 156.21 88.9) (end 156.21 91.44) (width 0.25) (layer F.Cu) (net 7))
 (segment (start 158.75 93.98) (end 158.75 99.06) (width 0.25) (layer F.Cu) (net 7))
 (segment (start 156.21 91.44) (end 158.75 93.98) (width 0.25) (layer F.Cu) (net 7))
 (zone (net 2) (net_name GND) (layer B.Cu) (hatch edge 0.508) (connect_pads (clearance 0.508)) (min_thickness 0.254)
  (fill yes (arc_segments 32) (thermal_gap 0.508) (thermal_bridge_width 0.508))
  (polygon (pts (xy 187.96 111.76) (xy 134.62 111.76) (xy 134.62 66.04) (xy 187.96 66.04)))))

